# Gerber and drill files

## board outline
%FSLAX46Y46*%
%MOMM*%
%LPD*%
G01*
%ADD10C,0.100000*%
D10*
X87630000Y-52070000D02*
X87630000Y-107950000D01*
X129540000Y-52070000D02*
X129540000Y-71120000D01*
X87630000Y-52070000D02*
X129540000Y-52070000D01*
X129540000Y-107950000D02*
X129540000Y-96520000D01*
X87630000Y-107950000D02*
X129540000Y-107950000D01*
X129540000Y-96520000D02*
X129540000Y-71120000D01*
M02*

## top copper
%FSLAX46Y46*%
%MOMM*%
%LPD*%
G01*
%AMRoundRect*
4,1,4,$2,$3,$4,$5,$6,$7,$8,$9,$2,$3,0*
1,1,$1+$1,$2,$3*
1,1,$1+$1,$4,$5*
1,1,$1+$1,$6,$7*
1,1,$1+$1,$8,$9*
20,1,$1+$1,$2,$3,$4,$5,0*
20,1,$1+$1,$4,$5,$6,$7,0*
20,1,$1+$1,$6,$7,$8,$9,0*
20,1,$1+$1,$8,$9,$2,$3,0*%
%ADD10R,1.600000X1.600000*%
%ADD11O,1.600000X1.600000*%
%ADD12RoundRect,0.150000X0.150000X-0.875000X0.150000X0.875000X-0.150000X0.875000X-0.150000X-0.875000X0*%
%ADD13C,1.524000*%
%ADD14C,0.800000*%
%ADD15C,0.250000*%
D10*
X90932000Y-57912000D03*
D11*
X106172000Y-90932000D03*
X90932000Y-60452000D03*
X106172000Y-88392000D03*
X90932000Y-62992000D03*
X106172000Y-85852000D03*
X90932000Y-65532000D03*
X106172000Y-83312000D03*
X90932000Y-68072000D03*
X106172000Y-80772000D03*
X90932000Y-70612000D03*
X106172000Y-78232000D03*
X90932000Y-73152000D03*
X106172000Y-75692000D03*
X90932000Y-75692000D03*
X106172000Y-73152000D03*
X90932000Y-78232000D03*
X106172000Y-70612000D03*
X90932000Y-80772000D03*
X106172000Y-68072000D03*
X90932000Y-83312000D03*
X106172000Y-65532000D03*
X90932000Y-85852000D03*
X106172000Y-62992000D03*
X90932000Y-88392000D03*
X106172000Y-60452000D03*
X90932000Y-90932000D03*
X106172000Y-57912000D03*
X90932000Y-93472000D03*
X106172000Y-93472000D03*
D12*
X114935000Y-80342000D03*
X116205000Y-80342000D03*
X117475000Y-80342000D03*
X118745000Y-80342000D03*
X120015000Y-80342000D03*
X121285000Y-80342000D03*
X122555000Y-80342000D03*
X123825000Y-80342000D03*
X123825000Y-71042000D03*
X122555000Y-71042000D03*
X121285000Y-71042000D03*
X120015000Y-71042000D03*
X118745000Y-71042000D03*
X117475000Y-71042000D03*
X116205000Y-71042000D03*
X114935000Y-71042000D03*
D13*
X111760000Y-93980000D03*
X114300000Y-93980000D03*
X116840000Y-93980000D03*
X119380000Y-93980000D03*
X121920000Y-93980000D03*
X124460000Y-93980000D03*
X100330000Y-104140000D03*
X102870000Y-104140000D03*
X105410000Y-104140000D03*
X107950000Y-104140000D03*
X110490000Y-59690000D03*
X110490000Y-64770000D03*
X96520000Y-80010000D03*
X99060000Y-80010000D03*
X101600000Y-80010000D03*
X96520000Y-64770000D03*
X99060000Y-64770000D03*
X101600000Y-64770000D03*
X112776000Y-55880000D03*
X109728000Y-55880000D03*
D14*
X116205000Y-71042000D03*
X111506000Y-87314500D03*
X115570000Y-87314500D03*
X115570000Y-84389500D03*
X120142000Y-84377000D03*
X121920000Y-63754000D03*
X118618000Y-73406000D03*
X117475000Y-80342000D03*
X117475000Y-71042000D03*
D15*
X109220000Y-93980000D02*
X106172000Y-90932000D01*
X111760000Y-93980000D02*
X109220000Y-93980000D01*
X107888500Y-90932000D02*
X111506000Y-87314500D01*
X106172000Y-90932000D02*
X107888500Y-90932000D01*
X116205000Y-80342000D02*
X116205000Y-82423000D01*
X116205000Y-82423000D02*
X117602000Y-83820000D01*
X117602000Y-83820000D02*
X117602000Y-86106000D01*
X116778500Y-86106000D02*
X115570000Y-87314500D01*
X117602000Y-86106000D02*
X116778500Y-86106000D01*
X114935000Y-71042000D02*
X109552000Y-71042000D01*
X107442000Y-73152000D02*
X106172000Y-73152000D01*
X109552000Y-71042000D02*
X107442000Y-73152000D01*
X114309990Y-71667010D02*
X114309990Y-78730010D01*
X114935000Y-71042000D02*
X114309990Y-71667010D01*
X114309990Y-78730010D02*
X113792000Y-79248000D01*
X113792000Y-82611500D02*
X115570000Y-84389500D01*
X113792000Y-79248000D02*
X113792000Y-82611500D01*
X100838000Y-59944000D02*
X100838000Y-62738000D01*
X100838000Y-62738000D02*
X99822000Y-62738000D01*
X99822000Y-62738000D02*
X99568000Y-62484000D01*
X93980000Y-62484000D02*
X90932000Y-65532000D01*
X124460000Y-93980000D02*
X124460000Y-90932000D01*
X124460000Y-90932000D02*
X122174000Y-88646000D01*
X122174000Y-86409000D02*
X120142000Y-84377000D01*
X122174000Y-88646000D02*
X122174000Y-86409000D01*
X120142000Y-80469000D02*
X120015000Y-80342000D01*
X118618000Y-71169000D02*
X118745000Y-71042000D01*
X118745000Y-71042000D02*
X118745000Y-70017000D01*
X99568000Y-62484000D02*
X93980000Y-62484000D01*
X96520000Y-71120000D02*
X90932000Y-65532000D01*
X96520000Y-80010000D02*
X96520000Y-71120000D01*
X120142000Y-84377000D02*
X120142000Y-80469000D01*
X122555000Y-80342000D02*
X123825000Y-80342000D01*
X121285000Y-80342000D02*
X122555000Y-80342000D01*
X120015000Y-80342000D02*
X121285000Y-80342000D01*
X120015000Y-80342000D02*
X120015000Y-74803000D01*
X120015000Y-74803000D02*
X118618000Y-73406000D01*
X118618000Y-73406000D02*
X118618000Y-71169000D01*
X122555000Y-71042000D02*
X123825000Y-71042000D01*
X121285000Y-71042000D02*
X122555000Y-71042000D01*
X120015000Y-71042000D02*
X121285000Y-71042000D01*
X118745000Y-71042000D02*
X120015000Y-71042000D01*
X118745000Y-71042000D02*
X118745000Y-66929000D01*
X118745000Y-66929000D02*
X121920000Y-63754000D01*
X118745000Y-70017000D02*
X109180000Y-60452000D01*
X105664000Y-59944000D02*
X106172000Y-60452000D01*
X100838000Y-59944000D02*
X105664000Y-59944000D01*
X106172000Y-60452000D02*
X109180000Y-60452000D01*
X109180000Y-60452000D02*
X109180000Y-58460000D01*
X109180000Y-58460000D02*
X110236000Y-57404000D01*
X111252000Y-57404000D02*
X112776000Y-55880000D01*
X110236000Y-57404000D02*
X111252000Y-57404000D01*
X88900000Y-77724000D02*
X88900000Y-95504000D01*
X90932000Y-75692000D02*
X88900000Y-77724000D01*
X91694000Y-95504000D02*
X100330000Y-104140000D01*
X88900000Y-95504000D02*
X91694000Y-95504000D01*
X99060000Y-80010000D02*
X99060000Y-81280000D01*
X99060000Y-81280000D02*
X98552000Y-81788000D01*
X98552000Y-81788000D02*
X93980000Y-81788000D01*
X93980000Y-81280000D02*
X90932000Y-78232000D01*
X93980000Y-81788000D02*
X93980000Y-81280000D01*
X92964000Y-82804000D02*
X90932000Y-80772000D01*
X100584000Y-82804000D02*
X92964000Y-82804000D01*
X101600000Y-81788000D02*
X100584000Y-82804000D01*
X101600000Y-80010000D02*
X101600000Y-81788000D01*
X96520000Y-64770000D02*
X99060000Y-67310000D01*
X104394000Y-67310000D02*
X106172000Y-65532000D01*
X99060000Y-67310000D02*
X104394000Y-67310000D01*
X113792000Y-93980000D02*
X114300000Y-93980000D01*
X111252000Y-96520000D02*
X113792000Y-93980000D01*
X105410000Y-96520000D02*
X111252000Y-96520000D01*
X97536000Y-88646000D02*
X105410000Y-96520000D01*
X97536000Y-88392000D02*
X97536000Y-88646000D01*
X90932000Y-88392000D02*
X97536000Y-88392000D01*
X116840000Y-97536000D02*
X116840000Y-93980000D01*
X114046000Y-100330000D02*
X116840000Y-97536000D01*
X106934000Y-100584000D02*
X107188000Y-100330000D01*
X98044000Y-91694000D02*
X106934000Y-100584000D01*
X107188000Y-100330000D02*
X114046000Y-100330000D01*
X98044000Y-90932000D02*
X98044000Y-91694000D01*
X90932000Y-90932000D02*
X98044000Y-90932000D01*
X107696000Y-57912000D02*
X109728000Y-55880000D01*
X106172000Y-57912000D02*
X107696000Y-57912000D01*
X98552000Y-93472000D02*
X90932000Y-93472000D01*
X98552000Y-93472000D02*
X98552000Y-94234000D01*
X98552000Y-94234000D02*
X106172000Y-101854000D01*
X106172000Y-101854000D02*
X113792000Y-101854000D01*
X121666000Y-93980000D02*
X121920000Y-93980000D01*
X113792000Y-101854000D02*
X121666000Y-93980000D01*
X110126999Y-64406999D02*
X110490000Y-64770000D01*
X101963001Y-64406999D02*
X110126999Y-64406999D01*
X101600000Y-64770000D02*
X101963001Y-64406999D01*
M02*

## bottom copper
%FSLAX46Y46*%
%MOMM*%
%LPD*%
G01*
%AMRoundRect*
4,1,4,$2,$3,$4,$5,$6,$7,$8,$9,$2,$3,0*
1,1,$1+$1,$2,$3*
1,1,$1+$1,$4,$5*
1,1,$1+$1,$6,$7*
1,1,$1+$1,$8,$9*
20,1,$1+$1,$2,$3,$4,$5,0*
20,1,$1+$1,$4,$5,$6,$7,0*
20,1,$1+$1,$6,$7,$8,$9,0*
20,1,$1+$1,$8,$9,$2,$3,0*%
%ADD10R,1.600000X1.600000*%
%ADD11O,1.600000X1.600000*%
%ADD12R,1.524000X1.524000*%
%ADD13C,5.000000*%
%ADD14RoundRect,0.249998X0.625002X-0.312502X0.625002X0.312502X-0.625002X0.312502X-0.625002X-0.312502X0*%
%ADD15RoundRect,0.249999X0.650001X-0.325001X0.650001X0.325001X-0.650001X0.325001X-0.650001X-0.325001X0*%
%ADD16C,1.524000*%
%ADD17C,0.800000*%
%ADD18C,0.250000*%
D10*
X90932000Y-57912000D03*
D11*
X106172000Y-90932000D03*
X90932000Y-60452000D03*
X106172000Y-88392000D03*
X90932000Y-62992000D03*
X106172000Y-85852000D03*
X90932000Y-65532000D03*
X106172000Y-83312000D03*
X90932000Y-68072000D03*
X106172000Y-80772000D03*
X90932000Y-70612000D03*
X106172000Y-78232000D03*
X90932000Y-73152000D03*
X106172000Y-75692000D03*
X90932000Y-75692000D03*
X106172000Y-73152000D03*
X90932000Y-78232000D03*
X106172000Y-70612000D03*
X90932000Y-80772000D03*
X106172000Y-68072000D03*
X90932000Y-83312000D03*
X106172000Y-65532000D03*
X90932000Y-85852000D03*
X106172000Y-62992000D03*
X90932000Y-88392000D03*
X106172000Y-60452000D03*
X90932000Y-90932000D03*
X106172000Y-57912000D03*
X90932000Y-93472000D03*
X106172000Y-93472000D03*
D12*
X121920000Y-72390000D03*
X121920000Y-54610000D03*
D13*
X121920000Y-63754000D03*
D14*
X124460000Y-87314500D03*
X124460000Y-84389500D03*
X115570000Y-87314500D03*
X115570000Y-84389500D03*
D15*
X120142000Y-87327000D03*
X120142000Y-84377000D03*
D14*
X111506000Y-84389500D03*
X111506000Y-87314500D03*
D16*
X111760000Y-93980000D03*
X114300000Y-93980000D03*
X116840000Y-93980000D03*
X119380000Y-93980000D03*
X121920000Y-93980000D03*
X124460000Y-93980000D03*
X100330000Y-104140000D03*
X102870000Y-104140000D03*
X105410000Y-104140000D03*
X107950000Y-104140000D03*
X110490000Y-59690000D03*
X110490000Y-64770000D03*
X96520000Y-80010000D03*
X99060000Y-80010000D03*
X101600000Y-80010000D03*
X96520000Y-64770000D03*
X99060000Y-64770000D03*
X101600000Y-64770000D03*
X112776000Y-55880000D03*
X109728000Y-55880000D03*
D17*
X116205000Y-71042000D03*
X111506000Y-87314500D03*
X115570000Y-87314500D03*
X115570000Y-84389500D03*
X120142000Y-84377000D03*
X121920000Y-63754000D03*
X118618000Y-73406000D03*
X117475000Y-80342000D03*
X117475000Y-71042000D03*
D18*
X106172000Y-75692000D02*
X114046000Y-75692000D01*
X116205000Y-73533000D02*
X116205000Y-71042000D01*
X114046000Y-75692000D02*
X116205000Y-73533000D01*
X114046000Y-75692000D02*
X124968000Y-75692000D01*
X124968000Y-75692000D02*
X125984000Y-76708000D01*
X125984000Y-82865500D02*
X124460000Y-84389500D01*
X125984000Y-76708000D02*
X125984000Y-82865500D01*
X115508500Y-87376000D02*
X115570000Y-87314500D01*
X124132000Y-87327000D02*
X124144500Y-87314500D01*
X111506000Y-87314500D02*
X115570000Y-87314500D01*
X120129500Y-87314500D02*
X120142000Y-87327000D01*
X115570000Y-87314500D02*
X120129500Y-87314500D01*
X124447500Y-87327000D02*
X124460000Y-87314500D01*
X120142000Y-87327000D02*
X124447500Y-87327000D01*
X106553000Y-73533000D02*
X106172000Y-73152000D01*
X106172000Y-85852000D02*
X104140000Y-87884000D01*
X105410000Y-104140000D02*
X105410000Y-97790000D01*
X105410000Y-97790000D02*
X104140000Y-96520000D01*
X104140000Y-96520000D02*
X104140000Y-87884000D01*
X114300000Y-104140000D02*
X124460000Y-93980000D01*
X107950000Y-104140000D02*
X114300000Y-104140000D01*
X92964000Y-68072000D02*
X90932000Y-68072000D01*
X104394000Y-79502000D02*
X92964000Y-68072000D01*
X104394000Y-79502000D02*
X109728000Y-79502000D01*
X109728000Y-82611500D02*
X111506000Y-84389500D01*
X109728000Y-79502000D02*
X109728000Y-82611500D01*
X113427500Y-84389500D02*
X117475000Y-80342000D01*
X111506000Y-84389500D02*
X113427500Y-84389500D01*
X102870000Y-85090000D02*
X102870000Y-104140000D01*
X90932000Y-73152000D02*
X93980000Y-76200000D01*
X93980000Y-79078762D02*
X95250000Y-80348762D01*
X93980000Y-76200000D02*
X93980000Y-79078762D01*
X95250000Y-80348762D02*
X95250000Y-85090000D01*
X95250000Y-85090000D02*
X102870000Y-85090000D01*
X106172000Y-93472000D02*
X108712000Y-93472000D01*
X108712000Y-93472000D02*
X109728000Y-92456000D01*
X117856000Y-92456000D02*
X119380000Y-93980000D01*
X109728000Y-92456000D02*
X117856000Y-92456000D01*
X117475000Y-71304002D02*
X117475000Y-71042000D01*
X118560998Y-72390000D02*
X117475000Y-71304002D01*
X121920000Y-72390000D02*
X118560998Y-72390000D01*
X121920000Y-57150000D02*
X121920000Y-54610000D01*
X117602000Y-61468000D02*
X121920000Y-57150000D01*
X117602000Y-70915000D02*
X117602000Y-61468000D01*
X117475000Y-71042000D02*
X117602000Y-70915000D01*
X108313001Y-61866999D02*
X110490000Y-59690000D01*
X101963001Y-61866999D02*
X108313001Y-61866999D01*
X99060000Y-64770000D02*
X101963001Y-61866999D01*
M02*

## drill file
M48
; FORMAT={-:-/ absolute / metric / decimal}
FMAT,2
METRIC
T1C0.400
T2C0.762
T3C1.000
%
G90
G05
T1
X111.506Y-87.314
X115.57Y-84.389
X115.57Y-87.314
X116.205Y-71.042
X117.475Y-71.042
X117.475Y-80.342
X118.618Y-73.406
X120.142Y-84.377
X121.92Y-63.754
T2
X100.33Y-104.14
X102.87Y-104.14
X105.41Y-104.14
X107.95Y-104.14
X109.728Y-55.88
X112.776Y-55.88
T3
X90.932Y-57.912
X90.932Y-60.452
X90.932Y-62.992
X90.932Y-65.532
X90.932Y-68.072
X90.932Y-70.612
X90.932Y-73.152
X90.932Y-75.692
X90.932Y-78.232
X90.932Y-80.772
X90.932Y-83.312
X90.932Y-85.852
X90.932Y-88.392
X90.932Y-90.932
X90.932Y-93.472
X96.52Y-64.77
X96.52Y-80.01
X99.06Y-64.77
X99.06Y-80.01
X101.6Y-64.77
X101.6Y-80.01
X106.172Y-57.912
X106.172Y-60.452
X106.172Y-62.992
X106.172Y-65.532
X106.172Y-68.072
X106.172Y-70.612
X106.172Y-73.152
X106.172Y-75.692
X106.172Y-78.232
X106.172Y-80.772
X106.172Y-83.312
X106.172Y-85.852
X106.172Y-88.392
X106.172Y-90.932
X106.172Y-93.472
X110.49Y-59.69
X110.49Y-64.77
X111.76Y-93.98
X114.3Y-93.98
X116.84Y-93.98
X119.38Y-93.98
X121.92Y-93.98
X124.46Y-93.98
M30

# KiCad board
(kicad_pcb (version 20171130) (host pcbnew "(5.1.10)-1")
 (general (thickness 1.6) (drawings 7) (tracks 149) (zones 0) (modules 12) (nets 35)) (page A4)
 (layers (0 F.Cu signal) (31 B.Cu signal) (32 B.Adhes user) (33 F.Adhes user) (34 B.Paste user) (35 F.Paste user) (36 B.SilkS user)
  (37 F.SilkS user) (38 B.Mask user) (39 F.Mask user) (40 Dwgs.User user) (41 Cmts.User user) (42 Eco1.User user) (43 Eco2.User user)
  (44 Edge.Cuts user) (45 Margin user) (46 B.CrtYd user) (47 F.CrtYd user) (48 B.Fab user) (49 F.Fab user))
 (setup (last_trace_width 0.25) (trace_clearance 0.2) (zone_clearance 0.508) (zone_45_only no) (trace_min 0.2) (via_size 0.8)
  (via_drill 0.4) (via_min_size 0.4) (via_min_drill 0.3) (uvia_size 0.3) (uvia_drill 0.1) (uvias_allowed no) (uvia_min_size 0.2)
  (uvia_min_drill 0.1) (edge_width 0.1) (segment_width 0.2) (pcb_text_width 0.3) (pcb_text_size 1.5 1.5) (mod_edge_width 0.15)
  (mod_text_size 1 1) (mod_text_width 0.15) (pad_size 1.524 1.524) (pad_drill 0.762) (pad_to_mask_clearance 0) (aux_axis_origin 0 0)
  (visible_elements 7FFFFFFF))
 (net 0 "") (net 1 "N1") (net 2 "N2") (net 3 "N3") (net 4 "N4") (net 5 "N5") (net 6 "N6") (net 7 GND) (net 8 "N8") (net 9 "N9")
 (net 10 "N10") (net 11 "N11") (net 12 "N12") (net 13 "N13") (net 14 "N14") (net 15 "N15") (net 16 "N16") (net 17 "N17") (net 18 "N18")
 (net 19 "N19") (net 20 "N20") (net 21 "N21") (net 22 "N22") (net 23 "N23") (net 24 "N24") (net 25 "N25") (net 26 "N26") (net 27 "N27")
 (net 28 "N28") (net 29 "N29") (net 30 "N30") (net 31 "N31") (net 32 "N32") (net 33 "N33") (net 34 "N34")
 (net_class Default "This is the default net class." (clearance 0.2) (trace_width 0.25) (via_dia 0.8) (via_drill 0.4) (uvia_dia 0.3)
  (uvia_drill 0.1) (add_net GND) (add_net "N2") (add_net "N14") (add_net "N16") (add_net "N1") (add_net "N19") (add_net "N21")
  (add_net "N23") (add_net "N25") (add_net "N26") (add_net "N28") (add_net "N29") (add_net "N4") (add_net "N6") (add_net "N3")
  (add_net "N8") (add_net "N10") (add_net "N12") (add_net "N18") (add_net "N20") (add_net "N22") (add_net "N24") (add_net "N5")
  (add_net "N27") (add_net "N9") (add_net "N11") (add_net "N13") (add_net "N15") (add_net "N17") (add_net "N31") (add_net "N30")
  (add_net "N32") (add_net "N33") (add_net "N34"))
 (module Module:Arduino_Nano (layer F.Cu) (at 90.932 57.912)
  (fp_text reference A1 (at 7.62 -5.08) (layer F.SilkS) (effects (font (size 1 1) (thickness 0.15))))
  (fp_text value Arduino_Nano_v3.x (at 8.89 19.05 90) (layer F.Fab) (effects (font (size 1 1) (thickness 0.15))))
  (pad 1 thru_hole rect (at 0 0) (size 1.6 1.6) (drill 1) (layers *.Cu *.Mask) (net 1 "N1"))
  (pad 17 thru_hole oval (at 15.24 33.02) (size 1.6 1.6) (drill 1) (layers *.Cu *.Mask) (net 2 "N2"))
  (pad 2 thru_hole oval (at 0 2.54) (size 1.6 1.6) (drill 1) (layers *.Cu *.Mask) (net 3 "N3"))
  (pad 18 thru_hole oval (at 15.24 30.48) (size 1.6 1.6) (drill 1) (layers *.Cu *.Mask) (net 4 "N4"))
  (pad 3 thru_hole oval (at 0 5.08) (size 1.6 1.6) (drill 1) (layers *.Cu *.Mask) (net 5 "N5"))
  (pad 19 thru_hole oval (at 15.24 27.94) (size 1.6 1.6) (drill 1) (layers *.Cu *.Mask) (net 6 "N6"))
  (pad 4 thru_hole oval (at 0 7.62) (size 1.6 1.6) (drill 1) (layers *.Cu *.Mask) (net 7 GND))
  (pad 20 thru_hole oval (at 15.24 25.4) (size 1.6 1.6) (drill 1) (layers *.Cu *.Mask) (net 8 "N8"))
  (pad 5 thru_hole oval (at 0 10.16) (size 1.6 1.6) (drill 1) (layers *.Cu *.Mask) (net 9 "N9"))
  (pad 21 thru_hole oval (at 15.24 22.86) (size 1.6 1.6) (drill 1) (layers *.Cu *.Mask) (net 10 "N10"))
  (pad 6 thru_hole oval (at 0 12.7) (size 1.6 1.6) (drill 1) (layers *.Cu *.Mask) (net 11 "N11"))
  (pad 22 thru_hole oval (at 15.24 20.32) (size 1.6 1.6) (drill 1) (layers *.Cu *.Mask) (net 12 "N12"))
  (pad 7 thru_hole oval (at 0 15.24) (size 1.6 1.6) (drill 1) (layers *.Cu *.Mask) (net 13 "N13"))
  (pad 23 thru_hole oval (at 15.24 17.78) (size 1.6 1.6) (drill 1) (layers *.Cu *.Mask) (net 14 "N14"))
  (pad 8 thru_hole oval (at 0 17.78) (size 1.6 1.6) (drill 1) (layers *.Cu *.Mask) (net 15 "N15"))
  (pad 24 thru_hole oval (at 15.24 15.24) (size 1.6 1.6) (drill 1) (layers *.Cu *.Mask) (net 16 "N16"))
  (pad 9 thru_hole oval (at 0 20.32) (size 1.6 1.6) (drill 1) (layers *.Cu *.Mask) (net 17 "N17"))
  (pad 25 thru_hole oval (at 15.24 12.7) (size 1.6 1.6) (drill 1) (layers *.Cu *.Mask) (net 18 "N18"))
  (pad 10 thru_hole oval (at 0 22.86) (size 1.6 1.6) (drill 1) (layers *.Cu *.Mask) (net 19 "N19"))
  (pad 26 thru_hole oval (at 15.24 10.16) (size 1.6 1.6) (drill 1) (layers *.Cu *.Mask) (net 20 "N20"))
  (pad 11 thru_hole oval (at 0 25.4) (size 1.6 1.6) (drill 1) (layers *.Cu *.Mask) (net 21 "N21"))
  (pad 27 thru_hole oval (at 15.24 7.62) (size 1.6 1.6) (drill 1) (layers *.Cu *.Mask) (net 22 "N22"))
  (pad 12 thru_hole oval (at 0 27.94) (size 1.6 1.6) (drill 1) (layers *.Cu *.Mask) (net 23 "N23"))
  (pad 28 thru_hole oval (at 15.24 5.08) (size 1.6 1.6) (drill 1) (layers *.Cu *.Mask) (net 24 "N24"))
  (pad 13 thru_hole oval (at 0 30.48) (size 1.6 1.6) (drill 1) (layers *.Cu *.Mask) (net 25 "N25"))
  (pad 29 thru_hole oval (at 15.24 2.54) (size 1.6 1.6) (drill 1) (layers *.Cu *.Mask) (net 7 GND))
  (pad 14 thru_hole oval (at 0 33.02) (size 1.6 1.6) (drill 1) (layers *.Cu *.Mask) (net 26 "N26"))
  (pad 30 thru_hole oval (at 15.24 0) (size 1.6 1.6) (drill 1) (layers *.Cu *.Mask) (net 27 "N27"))
  (pad 15 thru_hole oval (at 0 35.56) (size 1.6 1.6) (drill 1) (layers *.Cu *.Mask) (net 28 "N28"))
  (pad 16 thru_hole oval (at 15.24 35.56) (size 1.6 1.6) (drill 1) (layers *.Cu *.Mask) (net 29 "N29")))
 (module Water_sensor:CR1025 (layer B.Cu) (at 121.92 57.15)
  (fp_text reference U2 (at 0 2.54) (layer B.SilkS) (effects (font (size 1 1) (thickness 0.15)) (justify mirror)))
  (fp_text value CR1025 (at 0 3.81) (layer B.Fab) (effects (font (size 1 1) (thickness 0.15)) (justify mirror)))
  (pad 1 smd rect (at 0 15.24) (size 1.524 1.524) (layers B.Cu B.Paste B.Mask) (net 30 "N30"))
  (pad 2 smd rect (at 0 -2.54) (size 1.524 1.524) (layers B.Cu B.Paste B.Mask) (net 30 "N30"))
  (pad 3 smd circle (at 0 6.604) (size 5 5) (layers B.Cu B.Paste B.Mask) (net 7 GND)))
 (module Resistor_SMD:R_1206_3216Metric (layer B.Cu) (at 124.46 85.852 90)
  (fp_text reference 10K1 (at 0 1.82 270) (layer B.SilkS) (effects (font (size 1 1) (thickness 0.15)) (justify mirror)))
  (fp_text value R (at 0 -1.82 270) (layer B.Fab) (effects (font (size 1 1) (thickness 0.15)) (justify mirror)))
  (pad 1 smd roundrect (at -1.4625 0 90) (size 1.125 1.75) (layers B.Cu B.Paste B.Mask) (roundrect_rratio 0.2222204444444444) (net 2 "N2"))
  (pad 2 smd roundrect (at 1.4625 0 90) (size 1.125 1.75) (layers B.Cu B.Paste B.Mask) (roundrect_rratio 0.2222204444444444) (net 14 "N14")))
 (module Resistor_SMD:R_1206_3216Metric (layer B.Cu) (at 115.57 85.852 90)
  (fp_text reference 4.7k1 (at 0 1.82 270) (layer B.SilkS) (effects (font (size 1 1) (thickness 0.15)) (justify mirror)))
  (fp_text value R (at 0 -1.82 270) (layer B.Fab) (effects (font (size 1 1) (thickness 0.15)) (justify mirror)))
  (pad 1 smd roundrect (at -1.4625 0 90) (size 1.125 1.75) (layers B.Cu B.Paste B.Mask) (roundrect_rratio 0.2222204444444444) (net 2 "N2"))
  (pad 2 smd roundrect (at 1.4625 0 90) (size 1.125 1.75) (layers B.Cu B.Paste B.Mask) (roundrect_rratio 0.2222204444444444) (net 16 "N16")))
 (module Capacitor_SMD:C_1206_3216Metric (layer B.Cu) (at 120.142 85.852 90)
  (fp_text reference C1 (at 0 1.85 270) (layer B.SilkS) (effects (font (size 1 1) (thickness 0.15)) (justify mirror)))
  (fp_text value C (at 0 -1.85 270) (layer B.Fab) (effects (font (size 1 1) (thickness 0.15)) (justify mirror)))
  (pad 1 smd roundrect (at -1.475 0 90) (size 1.15 1.8) (layers B.Cu B.Paste B.Mask) (roundrect_rratio 0.2173904347826087) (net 2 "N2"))
  (pad 2 smd roundrect (at 1.475 0 90) (size 1.15 1.8) (layers B.Cu B.Paste B.Mask) (roundrect_rratio 0.2173904347826087) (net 7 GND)))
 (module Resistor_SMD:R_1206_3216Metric (layer B.Cu) (at 111.506 85.852 90)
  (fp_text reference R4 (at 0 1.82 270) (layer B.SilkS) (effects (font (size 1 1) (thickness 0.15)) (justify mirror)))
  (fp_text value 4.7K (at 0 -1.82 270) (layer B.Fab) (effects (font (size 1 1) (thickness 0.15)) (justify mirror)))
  (pad 2 smd roundrect (at 1.4625 0 90) (size 1.125 1.75) (layers B.Cu B.Paste B.Mask) (roundrect_rratio 0.2222204444444444) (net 9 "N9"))
  (pad 1 smd roundrect (at -1.4625 0 90) (size 1.125 1.75) (layers B.Cu B.Paste B.Mask) (roundrect_rratio 0.2222204444444444) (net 2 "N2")))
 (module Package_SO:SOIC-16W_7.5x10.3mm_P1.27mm (layer F.Cu) (at 119.38 75.692 90)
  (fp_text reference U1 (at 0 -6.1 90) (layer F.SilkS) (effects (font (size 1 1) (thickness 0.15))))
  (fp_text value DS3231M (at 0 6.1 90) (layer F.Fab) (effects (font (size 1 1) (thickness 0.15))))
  (pad 1 smd roundrect (at -4.65 -4.445 90) (size 2.05 0.6) (layers F.Cu F.Paste F.Mask) (roundrect_rratio 0.25) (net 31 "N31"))
  (pad 2 smd roundrect (at -4.65 -3.175 90) (size 2.05 0.6) (layers F.Cu F.Paste F.Mask) (roundrect_rratio 0.25) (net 2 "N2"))
  (pad 3 smd roundrect (at -4.65 -1.905 90) (size 2.05 0.6) (layers F.Cu F.Paste F.Mask) (roundrect_rratio 0.25) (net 9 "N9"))
  (pad 4 smd roundrect (at -4.65 -0.635 90) (size 2.05 0.6) (layers F.Cu F.Paste F.Mask) (roundrect_rratio 0.25) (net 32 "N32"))
  (pad 5 smd roundrect (at -4.65 0.635 90) (size 2.05 0.6) (layers F.Cu F.Paste F.Mask) (roundrect_rratio 0.25) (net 7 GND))
  (pad 6 smd roundrect (at -4.65 1.905 90) (size 2.05 0.6) (layers F.Cu F.Paste F.Mask) (roundrect_rratio 0.25) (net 7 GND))
  (pad 7 smd roundrect (at -4.65 3.175 90) (size 2.05 0.6) (layers F.Cu F.Paste F.Mask) (roundrect_rratio 0.25) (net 7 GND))
  (pad 8 smd roundrect (at -4.65 4.445 90) (size 2.05 0.6) (layers F.Cu F.Paste F.Mask) (roundrect_rratio 0.25) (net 7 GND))
  (pad 9 smd roundrect (at 4.65 4.445 90) (size 2.05 0.6) (layers F.Cu F.Paste F.Mask) (roundrect_rratio 0.25) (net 7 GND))
  (pad 10 smd roundrect (at 4.65 3.175 90) (size 2.05 0.6) (layers F.Cu F.Paste F.Mask) (roundrect_rratio 0.25) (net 7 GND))
  (pad 11 smd roundrect (at 4.65 1.905 90) (size 2.05 0.6) (layers F.Cu F.Paste F.Mask) (roundrect_rratio 0.25) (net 7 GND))
  (pad 12 smd roundrect (at 4.65 0.635 90) (size 2.05 0.6) (layers F.Cu F.Paste F.Mask) (roundrect_rratio 0.25) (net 7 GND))
  (pad 13 smd roundrect (at 4.65 -0.635 90) (size 2.05 0.6) (layers F.Cu F.Paste F.Mask) (roundrect_rratio 0.25) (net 7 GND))
  (pad 14 smd roundrect (at 4.65 -1.905 90) (size 2.05 0.6) (layers F.Cu F.Paste F.Mask) (roundrect_rratio 0.25) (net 30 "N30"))
  (pad 15 smd roundrect (at 4.65 -3.175 90) (size 2.05 0.6) (layers F.Cu F.Paste F.Mask) (roundrect_rratio 0.25) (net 14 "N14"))
  (pad 16 smd roundrect (at 4.65 -4.445 90) (size 2.05 0.6) (layers F.Cu F.Paste F.Mask) (roundrect_rratio 0.25) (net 16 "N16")))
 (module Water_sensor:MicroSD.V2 (layer F.Cu) (at 119.38 91.44)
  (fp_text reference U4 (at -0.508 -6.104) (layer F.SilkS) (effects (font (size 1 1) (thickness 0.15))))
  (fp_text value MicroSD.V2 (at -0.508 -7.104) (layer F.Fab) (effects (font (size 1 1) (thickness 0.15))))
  (pad 1 thru_hole circle (at -7.62 2.54) (size 1.524 1.524) (drill 1) (layers *.Cu *.Mask) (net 2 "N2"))
  (pad 2 thru_hole circle (at -5.08 2.54) (size 1.524 1.524) (drill 1) (layers *.Cu *.Mask) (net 25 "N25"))
  (pad 3 thru_hole circle (at -2.54 2.54) (size 1.524 1.524) (drill 1) (layers *.Cu *.Mask) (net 26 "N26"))
  (pad 4 thru_hole circle (at 0 2.54) (size 1.524 1.524) (drill 1) (layers *.Cu *.Mask) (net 29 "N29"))
  (pad 5 thru_hole circle (at 2.54 2.54) (size 1.524 1.524) (drill 1) (layers *.Cu *.Mask) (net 28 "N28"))
  (pad 6 thru_hole circle (at 5.08 2.54) (size 1.524 1.524) (drill 1) (layers *.Cu *.Mask) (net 7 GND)))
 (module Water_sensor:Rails (layer F.Cu) (at 104.14 101.6)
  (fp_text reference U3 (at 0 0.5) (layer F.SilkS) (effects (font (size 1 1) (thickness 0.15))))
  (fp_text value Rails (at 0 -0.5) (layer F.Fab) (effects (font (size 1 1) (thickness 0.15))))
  (pad 1 thru_hole circle (at -3.81 2.54) (size 1.524 1.524) (drill 0.762) (layers *.Cu *.Mask) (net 15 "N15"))
  (pad 2 thru_hole circle (at -1.27 2.54) (size 1.524 1.524) (drill 0.762) (layers *.Cu *.Mask) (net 13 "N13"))
  (pad 3 thru_hole circle (at 1.27 2.54) (size 1.524 1.524) (drill 0.762) (layers *.Cu *.Mask) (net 6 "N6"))
  (pad 4 thru_hole circle (at 3.81 2.54) (size 1.524 1.524) (drill 0.762) (layers *.Cu *.Mask) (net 7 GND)))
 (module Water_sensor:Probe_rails (layer F.Cu) (at 113.03 62.23 270)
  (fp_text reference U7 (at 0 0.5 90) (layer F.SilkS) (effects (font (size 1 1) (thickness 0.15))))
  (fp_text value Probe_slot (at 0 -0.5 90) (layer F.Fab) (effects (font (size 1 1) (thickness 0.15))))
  (pad 1 thru_hole circle (at -2.54 2.54 270) (size 1.524 1.524) (drill 1) (layers *.Cu *.Mask) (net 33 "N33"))
  (pad 2 thru_hole circle (at 2.54 2.54 270) (size 1.524 1.524) (drill 1) (layers *.Cu *.Mask) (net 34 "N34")))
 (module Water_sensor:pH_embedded (layer B.Cu) (at 99.06 67.31)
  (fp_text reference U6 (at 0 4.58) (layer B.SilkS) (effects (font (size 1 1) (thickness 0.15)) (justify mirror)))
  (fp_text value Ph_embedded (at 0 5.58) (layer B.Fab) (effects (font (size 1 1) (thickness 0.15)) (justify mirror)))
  (pad 1 thru_hole circle (at -2.54 12.7) (size 1.524 1.524) (drill 1) (layers *.Cu *.Mask) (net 7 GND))
  (pad 2 thru_hole circle (at 0 12.7) (size 1.524 1.524) (drill 1) (layers *.Cu *.Mask) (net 17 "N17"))
  (pad 3 thru_hole circle (at 2.54 12.7) (size 1.524 1.524) (drill 1) (layers *.Cu *.Mask) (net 19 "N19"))
  (pad 4 thru_hole circle (at -2.54 -2.54) (size 1.524 1.524) (drill 1) (layers *.Cu *.Mask) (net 22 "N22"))
  (pad 5 thru_hole circle (at 0 -2.54) (size 1.524 1.524) (drill 1) (layers *.Cu *.Mask) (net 33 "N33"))
  (pad 6 thru_hole circle (at 2.54 -2.54) (size 1.524 1.524) (drill 1) (layers *.Cu *.Mask) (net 34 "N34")))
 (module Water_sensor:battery (layer F.Cu) (at 111.252 53.848)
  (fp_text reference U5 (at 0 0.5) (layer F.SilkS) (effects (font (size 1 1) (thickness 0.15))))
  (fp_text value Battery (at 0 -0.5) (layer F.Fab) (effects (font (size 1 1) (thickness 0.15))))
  (pad 2 thru_hole circle (at 1.524 2.032) (size 1.524 1.524) (drill 0.762) (layers *.Cu *.Mask) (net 7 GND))
  (pad 1 thru_hole circle (at -1.524 2.032) (size 1.524 1.524) (drill 0.762) (layers *.Cu *.Mask) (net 27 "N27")))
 (gr_line (start 87.63 52.07) (end 87.63 107.95) (layer Edge.Cuts) (width 0.1))
 (gr_line (start 129.54 52.07) (end 129.54 71.12) (layer Edge.Cuts) (width 0.1))
 (gr_line (start 87.63 52.07) (end 129.54 52.07) (layer Edge.Cuts) (width 0.1))
 (gr_line (start 129.54 107.95) (end 129.54 96.52) (layer Edge.Cuts) (width 0.1))
 (gr_line (start 87.63 107.95) (end 129.54 107.95) (layer Edge.Cuts) (width 0.1))
 (gr_line (start 129.54 96.52) (end 129.54 71.12) (layer Edge.Cuts) (width 0.1))
 (segment (start 106.172 75.692) (end 114.046 75.692) (width 0.25) (layer B.Cu) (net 14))
 (via (at 116.205 71.042) (size 0.8) (drill 0.4) (layers F.Cu B.Cu) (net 14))
 (segment (start 116.205 73.533) (end 116.205 71.042) (width 0.25) (layer B.Cu) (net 14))
 (segment (start 114.046 75.692) (end 116.205 73.533) (width 0.25) (layer B.Cu) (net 14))
 (segment (start 114.046 75.692) (end 124.968 75.692) (width 0.25) (layer B.Cu) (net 14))
 (segment (start 124.968 75.692) (end 125.984 76.708) (width 0.25) (layer B.Cu) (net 14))
 (segment (start 125.984 82.8655) (end 124.46 84.3895) (width 0.25) (layer B.Cu) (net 14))
 (segment (start 125.984 76.708) (end 125.984 82.8655) (width 0.25) (layer B.Cu) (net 14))
 (segment (start 115.5085 87.376) (end 115.57 87.3145) (width 0.25) (layer B.Cu) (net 2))
 (segment (start 124.132 87.327) (end 124.1445 87.3145) (width 0.25) (layer B.Cu) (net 2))
 (segment (start 109.22 93.98) (end 106.172 90.932) (width 0.25) (layer F.Cu) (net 2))
 (segment (start 111.76 93.98) (end 109.22 93.98) (width 0.25) (layer F.Cu) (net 2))
 (via (at 111.506 87.3145) (size 0.8) (drill 0.4) (layers F.Cu B.Cu) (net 2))
 (segment (start 107.8885 90.932) (end 111.506 87.3145) (width 0.25) (layer F.Cu) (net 2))
 (segment (start 106.172 90.932) (end 107.8885 90.932) (width 0.25) (layer F.Cu) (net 2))
 (segment (start 111.506 87.3145) (end 115.57 87.3145) (width 0.25) (layer B.Cu) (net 2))
 (segment (start 120.1295 87.3145) (end 120.142 87.327) (width 0.25) (layer B.Cu) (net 2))
 (segment (start 115.57 87.3145) (end 120.1295 87.3145) (width 0.25) (layer B.Cu) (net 2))
 (segment (start 124.4475 87.327) (end 124.46 87.3145) (width 0.25) (layer B.Cu) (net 2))
 (segment (start 120.142 87.327) (end 124.4475 87.327) (width 0.25) (layer B.Cu) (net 2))
 (segment (start 116.205 80.342) (end 116.205 82.423) (width 0.25) (layer F.Cu) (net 2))
 (segment (start 116.205 82.423) (end 117.602 83.82) (width 0.25) (layer F.Cu) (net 2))
 (segment (start 117.602 83.82) (end 117.602 86.106) (width 0.25) (layer F.Cu) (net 2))
 (via (at 115.57 87.3145) (size 0.8) (drill 0.4) (layers F.Cu B.Cu) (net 2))
 (segment (start 116.7785 86.106) (end 115.57 87.3145) (width 0.25) (layer F.Cu) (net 2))
 (segment (start 117.602 86.106) (end 116.7785 86.106) (width 0.25) (layer F.Cu) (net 2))
 (segment (start 106.553 73.533) (end 106.172 73.152) (width 0.25) (layer B.Cu) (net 16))
 (segment (start 114.935 71.042) (end 109.552 71.042) (width 0.25) (layer F.Cu) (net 16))
 (segment (start 107.442 73.152) (end 106.172 73.152) (width 0.25) (layer F.Cu) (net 16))
 (segment (start 109.552 71.042) (end 107.442 73.152) (width 0.25) (layer F.Cu) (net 16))
 (segment (start 114.30999 71.66701) (end 114.30999 78.73001) (width 0.25) (layer F.Cu) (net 16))
 (segment (start 114.935 71.042) (end 114.30999 71.66701) (width 0.25) (layer F.Cu) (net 16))
 (segment (start 114.30999 78.73001) (end 113.792 79.248) (width 0.25) (layer F.Cu) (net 16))
 (via (at 115.57 84.3895) (size 0.8) (drill 0.4) (layers F.Cu B.Cu) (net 16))
 (segment (start 113.792 82.6115) (end 115.57 84.3895) (width 0.25) (layer F.Cu) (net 16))
 (segment (start 113.792 79.248) (end 113.792 82.6115) (width 0.25) (layer F.Cu) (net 16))
 (segment (start 106.172 85.852) (end 104.14 87.884) (width 0.25) (layer B.Cu) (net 6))
 (segment (start 105.41 104.14) (end 105.41 97.79) (width 0.25) (layer B.Cu) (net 6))
 (segment (start 105.41 97.79) (end 104.14 96.52) (width 0.25) (layer B.Cu) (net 6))
 (segment (start 104.14 96.52) (end 104.14 87.884) (width 0.25) (layer B.Cu) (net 6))
 (segment (start 100.838 59.944) (end 100.838 62.738) (width 0.25) (layer F.Cu) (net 7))
 (segment (start 100.838 62.738) (end 99.822 62.738) (width 0.25) (layer F.Cu) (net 7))
 (segment (start 99.822 62.738) (end 99.568 62.484) (width 0.25) (layer F.Cu) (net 7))
 (segment (start 93.98 62.484) (end 90.932 65.532) (width 0.25) (layer F.Cu) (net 7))
 (segment (start 124.46 93.98) (end 124.46 90.932) (width 0.25) (layer F.Cu) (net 7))
 (segment (start 124.46 90.932) (end 122.174 88.646) (width 0.25) (layer F.Cu) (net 7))
 (via (at 120.142 84.377) (size 0.8) (drill 0.4) (layers F.Cu B.Cu) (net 7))
 (segment (start 122.174 86.409) (end 120.142 84.377) (width 0.25) (layer F.Cu) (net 7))
 (segment (start 122.174 88.646) (end 122.174 86.409) (width 0.25) (layer F.Cu) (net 7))
 (segment (start 120.142 80.469) (end 120.015 80.342) (width 0.25) (layer F.Cu) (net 7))
 (segment (start 118.618 71.169) (end 118.745 71.042) (width 0.25) (layer F.Cu) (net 7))
 (segment (start 118.745 71.042) (end 118.745 70.017) (width 0.25) (layer F.Cu) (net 7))
 (segment (start 114.3 104.14) (end 124.46 93.98) (width 0.25) (layer B.Cu) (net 7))
 (segment (start 107.95 104.14) (end 114.3 104.14) (width 0.25) (layer B.Cu) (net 7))
 (segment (start 99.568 62.484) (end 93.98 62.484) (width 0.25) (layer F.Cu) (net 7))
 (segment (start 96.52 71.12) (end 90.932 65.532) (width 0.25) (layer F.Cu) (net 7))
 (segment (start 96.52 80.01) (end 96.52 71.12) (width 0.25) (layer F.Cu) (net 7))
 (via (at 121.92 63.754) (size 0.8) (drill 0.4) (layers F.Cu B.Cu) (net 7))
 (segment (start 120.142 84.377) (end 120.142 80.469) (width 0.25) (layer F.Cu) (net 7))
 (segment (start 122.555 80.342) (end 123.825 80.342) (width 0.25) (layer F.Cu) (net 7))
 (segment (start 121.285 80.342) (end 122.555 80.342) (width 0.25) (layer F.Cu) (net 7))
 (segment (start 120.015 80.342) (end 121.285 80.342) (width 0.25) (layer F.Cu) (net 7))
 (segment (start 120.015 80.342) (end 120.015 74.803) (width 0.25) (layer F.Cu) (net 7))
 (segment (start 120.015 74.803) (end 118.618 73.406) (width 0.25) (layer F.Cu) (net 7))
 (via (at 118.618 73.406) (size 0.8) (drill 0.4) (layers F.Cu B.Cu) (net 7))
 (segment (start 118.618 73.406) (end 118.618 71.169) (width 0.25) (layer F.Cu) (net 7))
 (segment (start 122.555 71.042) (end 123.825 71.042) (width 0.25) (layer F.Cu) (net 7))
 (segment (start 121.285 71.042) (end 122.555 71.042) (width 0.25) (layer F.Cu) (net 7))
 (segment (start 120.015 71.042) (end 121.285 71.042) (width 0.25) (layer F.Cu) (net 7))
 (segment (start 118.745 71.042) (end 120.015 71.042) (width 0.25) (layer F.Cu) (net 7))
 (segment (start 118.745 71.042) (end 118.745 66.929) (width 0.25) (layer F.Cu) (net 7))
 (segment (start 118.745 66.929) (end 121.92 63.754) (width 0.25) (layer F.Cu) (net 7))
 (segment (start 118.745 70.017) (end 109.18 60.452) (width 0.25) (layer F.Cu) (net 7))
 (segment (start 105.664 59.944) (end 106.172 60.452) (width 0.25) (layer F.Cu) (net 7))
 (segment (start 100.838 59.944) (end 105.664 59.944) (width 0.25) (layer F.Cu) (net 7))
 (segment (start 106.172 60.452) (end 109.18 60.452) (width 0.25) (layer F.Cu) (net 7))
 (segment (start 109.18 60.452) (end 109.18 58.46) (width 0.25) (layer F.Cu) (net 7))
 (segment (start 109.18 58.46) (end 110.236 57.404) (width 0.25) (layer F.Cu) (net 7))
 (segment (start 111.252 57.404) (end 112.776 55.88) (width 0.25) (layer F.Cu) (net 7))
 (segment (start 110.236 57.404) (end 111.252 57.404) (width 0.25) (layer F.Cu) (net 7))
 (segment (start 92.964 68.072) (end 90.932 68.072) (width 0.25) (layer B.Cu) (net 9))
 (segment (start 104.394 79.502) (end 92.964 68.072) (width 0.25) (layer B.Cu) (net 9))
 (segment (start 104.394 79.502) (end 109.728 79.502) (width 0.25) (layer B.Cu) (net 9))
 (segment (start 109.728 82.6115) (end 111.506 84.3895) (width 0.25) (layer B.Cu) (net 9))
 (segment (start 109.728 79.502) (end 109.728 82.6115) (width 0.25) (layer B.Cu) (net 9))
 (via (at 117.475 80.342) (size 0.8) (drill 0.4) (layers F.Cu B.Cu) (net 9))
 (segment (start 113.4275 84.3895) (end 117.475 80.342) (width 0.25) (layer B.Cu) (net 9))
 (segment (start 111.506 84.3895) (end 113.4275 84.3895) (width 0.25) (layer B.Cu) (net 9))
 (segment (start 102.87 85.09) (end 102.87 104.14) (width 0.25) (layer B.Cu) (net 13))
 (segment (start 90.932 73.152) (end 93.98 76.2) (width 0.25) (layer B.Cu) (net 13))
 (segment (start 93.98 79.078762) (end 95.25 80.348762) (width 0.25) (layer B.Cu) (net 13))
 (segment (start 93.98 76.2) (end 93.98 79.078762) (width 0.25) (layer B.Cu) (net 13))
 (segment (start 95.25 80.348762) (end 95.25 85.09) (width 0.25) (layer B.Cu) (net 13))
 (segment (start 95.25 85.09) (end 102.87 85.09) (width 0.25) (layer B.Cu) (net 13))
 (segment (start 88.9 77.724) (end 88.9 95.504) (width 0.25) (layer F.Cu) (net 15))
 (segment (start 90.932 75.692) (end 88.9 77.724) (width 0.25) (layer F.Cu) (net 15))
 (segment (start 91.694 95.504) (end 100.33 104.14) (width 0.25) (layer F.Cu) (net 15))
 (segment (start 88.9 95.504) (end 91.694 95.504) (width 0.25) (layer F.Cu) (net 15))
 (segment (start 99.06 80.01) (end 99.06 81.28) (width 0.25) (layer F.Cu) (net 17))
 (segment (start 99.06 81.28) (end 98.552 81.788) (width 0.25) (layer F.Cu) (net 17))
 (segment (start 98.552 81.788) (end 93.98 81.788) (width 0.25) (layer F.Cu) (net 17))
 (segment (start 93.98 81.28) (end 90.932 78.232) (width 0.25) (layer F.Cu) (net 17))
 (segment (start 93.98 81.788) (end 93.98 81.28) (width 0.25) (layer F.Cu) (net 17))
 (segment (start 92.964 82.804) (end 90.932 80.772) (width 0.25) (layer F.Cu) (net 19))
 (segment (start 100.584 82.804) (end 92.964 82.804) (width 0.25) (layer F.Cu) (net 19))
 (segment (start 101.6 81.788) (end 100.584 82.804) (width 0.25) (layer F.Cu) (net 19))
 (segment (start 101.6 80.01) (end 101.6 81.788) (width 0.25) (layer F.Cu) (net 19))
 (segment (start 96.52 64.77) (end 99.06 67.31) (width 0.25) (layer F.Cu) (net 22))
 (segment (start 104.394 67.31) (end 106.172 65.532) (width 0.25) (layer F.Cu) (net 22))
 (segment (start 99.06 67.31) (end 104.394 67.31) (width 0.25) (layer F.Cu) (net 22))
 (segment (start 113.792 93.98) (end 114.3 93.98) (width 0.25) (layer F.Cu) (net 25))
 (segment (start 111.252 96.52) (end 113.792 93.98) (width 0.25) (layer F.Cu) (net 25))
 (segment (start 105.41 96.52) (end 111.252 96.52) (width 0.25) (layer F.Cu) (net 25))
 (segment (start 97.536 88.646) (end 105.41 96.52) (width 0.25) (layer F.Cu) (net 25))
 (segment (start 97.536 88.392) (end 97.536 88.646) (width 0.25) (layer F.Cu) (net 25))
 (segment (start 90.932 88.392) (end 97.536 88.392) (width 0.25) (layer F.Cu) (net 25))
 (segment (start 116.84 97.536) (end 116.84 93.98) (width 0.25) (layer F.Cu) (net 26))
 (segment (start 114.046 100.33) (end 116.84 97.536) (width 0.25) (layer F.Cu) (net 26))
 (segment (start 106.934 100.584) (end 107.188 100.33) (width 0.25) (layer F.Cu) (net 26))
 (segment (start 98.044 91.694) (end 106.934 100.584) (width 0.25) (layer F.Cu) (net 26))
 (segment (start 107.188 100.33) (end 114.046 100.33) (width 0.25) (layer F.Cu) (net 26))
 (segment (start 98.044 90.932) (end 98.044 91.694) (width 0.25) (layer F.Cu) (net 26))
 (segment (start 90.932 90.932) (end 98.044 90.932) (width 0.25) (layer F.Cu) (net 26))
 (segment (start 107.696 57.912) (end 109.728 55.88) (width 0.25) (layer F.Cu) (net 27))
 (segment (start 106.172 57.912) (end 107.696 57.912) (width 0.25) (layer F.Cu) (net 27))
 (segment (start 98.552 93.472) (end 90.932 93.472) (width 0.25) (layer F.Cu) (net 28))
 (segment (start 98.552 93.472) (end 98.552 94.234) (width 0.25) (layer F.Cu) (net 28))
 (segment (start 98.552 94.234) (end 106.172 101.854) (width 0.25) (layer F.Cu) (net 28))
 (segment (start 106.172 101.854) (end 113.792 101.854) (width 0.25) (layer F.Cu) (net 28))
 (segment (start 121.666 93.98) (end 121.92 93.98) (width 0.25) (layer F.Cu) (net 28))
 (segment (start 113.792 101.854) (end 121.666 93.98) (width 0.25) (layer F.Cu) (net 28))
 (segment (start 106.172 93.472) (end 108.712 93.472) (width 0.25) (layer B.Cu) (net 29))
 (segment (start 108.712 93.472) (end 109.728 92.456) (width 0.25) (layer B.Cu) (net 29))
 (segment (start 117.856 92.456) (end 119.38 93.98) (width 0.25) (layer B.Cu) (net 29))
 (segment (start 109.728 92.456) (end 117.856 92.456) (width 0.25) (layer B.Cu) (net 29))
 (via (at 117.475 71.042) (size 0.8) (drill 0.4) (layers F.Cu B.Cu) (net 30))
 (segment (start 117.475 71.304002) (end 117.475 71.042) (width 0.25) (layer B.Cu) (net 30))
 (segment (start 118.560998 72.39) (end 117.475 71.304002) (width 0.25) (layer B.Cu) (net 30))
 (segment (start 121.92 72.39) (end 118.560998 72.39) (width 0.25) (layer B.Cu) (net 30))
 (segment (start 121.92 57.15) (end 121.92 54.61) (width 0.25) (layer B.Cu) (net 30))
 (segment (start 117.602 61.468) (end 121.92 57.15) (width 0.25) (layer B.Cu) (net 30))
 (segment (start 117.602 70.915) (end 117.602 61.468) (width 0.25) (layer B.Cu) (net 30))
 (segment (start 117.475 71.042) (end 117.602 70.915) (width 0.25) (layer B.Cu) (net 30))
 (segment (start 108.313001 61.866999) (end 110.49 59.69) (width 0.25) (layer B.Cu) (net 33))
 (segment (start 101.963001 61.866999) (end 108.313001 61.866999) (width 0.25) (layer B.Cu) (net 33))
 (segment (start 99.06 64.77) (end 101.963001 61.866999) (width 0.25) (layer B.Cu) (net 33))
 (segment (start 110.126999 64.406999) (end 110.49 64.77) (width 0.25) (layer F.Cu) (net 34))
 (segment (start 101.963001 64.406999) (end 110.126999 64.406999) (width 0.25) (layer F.Cu) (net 34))
 (segment (start 101.6 64.77) (end 101.963001 64.406999) (width 0.25) (layer F.Cu) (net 34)))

